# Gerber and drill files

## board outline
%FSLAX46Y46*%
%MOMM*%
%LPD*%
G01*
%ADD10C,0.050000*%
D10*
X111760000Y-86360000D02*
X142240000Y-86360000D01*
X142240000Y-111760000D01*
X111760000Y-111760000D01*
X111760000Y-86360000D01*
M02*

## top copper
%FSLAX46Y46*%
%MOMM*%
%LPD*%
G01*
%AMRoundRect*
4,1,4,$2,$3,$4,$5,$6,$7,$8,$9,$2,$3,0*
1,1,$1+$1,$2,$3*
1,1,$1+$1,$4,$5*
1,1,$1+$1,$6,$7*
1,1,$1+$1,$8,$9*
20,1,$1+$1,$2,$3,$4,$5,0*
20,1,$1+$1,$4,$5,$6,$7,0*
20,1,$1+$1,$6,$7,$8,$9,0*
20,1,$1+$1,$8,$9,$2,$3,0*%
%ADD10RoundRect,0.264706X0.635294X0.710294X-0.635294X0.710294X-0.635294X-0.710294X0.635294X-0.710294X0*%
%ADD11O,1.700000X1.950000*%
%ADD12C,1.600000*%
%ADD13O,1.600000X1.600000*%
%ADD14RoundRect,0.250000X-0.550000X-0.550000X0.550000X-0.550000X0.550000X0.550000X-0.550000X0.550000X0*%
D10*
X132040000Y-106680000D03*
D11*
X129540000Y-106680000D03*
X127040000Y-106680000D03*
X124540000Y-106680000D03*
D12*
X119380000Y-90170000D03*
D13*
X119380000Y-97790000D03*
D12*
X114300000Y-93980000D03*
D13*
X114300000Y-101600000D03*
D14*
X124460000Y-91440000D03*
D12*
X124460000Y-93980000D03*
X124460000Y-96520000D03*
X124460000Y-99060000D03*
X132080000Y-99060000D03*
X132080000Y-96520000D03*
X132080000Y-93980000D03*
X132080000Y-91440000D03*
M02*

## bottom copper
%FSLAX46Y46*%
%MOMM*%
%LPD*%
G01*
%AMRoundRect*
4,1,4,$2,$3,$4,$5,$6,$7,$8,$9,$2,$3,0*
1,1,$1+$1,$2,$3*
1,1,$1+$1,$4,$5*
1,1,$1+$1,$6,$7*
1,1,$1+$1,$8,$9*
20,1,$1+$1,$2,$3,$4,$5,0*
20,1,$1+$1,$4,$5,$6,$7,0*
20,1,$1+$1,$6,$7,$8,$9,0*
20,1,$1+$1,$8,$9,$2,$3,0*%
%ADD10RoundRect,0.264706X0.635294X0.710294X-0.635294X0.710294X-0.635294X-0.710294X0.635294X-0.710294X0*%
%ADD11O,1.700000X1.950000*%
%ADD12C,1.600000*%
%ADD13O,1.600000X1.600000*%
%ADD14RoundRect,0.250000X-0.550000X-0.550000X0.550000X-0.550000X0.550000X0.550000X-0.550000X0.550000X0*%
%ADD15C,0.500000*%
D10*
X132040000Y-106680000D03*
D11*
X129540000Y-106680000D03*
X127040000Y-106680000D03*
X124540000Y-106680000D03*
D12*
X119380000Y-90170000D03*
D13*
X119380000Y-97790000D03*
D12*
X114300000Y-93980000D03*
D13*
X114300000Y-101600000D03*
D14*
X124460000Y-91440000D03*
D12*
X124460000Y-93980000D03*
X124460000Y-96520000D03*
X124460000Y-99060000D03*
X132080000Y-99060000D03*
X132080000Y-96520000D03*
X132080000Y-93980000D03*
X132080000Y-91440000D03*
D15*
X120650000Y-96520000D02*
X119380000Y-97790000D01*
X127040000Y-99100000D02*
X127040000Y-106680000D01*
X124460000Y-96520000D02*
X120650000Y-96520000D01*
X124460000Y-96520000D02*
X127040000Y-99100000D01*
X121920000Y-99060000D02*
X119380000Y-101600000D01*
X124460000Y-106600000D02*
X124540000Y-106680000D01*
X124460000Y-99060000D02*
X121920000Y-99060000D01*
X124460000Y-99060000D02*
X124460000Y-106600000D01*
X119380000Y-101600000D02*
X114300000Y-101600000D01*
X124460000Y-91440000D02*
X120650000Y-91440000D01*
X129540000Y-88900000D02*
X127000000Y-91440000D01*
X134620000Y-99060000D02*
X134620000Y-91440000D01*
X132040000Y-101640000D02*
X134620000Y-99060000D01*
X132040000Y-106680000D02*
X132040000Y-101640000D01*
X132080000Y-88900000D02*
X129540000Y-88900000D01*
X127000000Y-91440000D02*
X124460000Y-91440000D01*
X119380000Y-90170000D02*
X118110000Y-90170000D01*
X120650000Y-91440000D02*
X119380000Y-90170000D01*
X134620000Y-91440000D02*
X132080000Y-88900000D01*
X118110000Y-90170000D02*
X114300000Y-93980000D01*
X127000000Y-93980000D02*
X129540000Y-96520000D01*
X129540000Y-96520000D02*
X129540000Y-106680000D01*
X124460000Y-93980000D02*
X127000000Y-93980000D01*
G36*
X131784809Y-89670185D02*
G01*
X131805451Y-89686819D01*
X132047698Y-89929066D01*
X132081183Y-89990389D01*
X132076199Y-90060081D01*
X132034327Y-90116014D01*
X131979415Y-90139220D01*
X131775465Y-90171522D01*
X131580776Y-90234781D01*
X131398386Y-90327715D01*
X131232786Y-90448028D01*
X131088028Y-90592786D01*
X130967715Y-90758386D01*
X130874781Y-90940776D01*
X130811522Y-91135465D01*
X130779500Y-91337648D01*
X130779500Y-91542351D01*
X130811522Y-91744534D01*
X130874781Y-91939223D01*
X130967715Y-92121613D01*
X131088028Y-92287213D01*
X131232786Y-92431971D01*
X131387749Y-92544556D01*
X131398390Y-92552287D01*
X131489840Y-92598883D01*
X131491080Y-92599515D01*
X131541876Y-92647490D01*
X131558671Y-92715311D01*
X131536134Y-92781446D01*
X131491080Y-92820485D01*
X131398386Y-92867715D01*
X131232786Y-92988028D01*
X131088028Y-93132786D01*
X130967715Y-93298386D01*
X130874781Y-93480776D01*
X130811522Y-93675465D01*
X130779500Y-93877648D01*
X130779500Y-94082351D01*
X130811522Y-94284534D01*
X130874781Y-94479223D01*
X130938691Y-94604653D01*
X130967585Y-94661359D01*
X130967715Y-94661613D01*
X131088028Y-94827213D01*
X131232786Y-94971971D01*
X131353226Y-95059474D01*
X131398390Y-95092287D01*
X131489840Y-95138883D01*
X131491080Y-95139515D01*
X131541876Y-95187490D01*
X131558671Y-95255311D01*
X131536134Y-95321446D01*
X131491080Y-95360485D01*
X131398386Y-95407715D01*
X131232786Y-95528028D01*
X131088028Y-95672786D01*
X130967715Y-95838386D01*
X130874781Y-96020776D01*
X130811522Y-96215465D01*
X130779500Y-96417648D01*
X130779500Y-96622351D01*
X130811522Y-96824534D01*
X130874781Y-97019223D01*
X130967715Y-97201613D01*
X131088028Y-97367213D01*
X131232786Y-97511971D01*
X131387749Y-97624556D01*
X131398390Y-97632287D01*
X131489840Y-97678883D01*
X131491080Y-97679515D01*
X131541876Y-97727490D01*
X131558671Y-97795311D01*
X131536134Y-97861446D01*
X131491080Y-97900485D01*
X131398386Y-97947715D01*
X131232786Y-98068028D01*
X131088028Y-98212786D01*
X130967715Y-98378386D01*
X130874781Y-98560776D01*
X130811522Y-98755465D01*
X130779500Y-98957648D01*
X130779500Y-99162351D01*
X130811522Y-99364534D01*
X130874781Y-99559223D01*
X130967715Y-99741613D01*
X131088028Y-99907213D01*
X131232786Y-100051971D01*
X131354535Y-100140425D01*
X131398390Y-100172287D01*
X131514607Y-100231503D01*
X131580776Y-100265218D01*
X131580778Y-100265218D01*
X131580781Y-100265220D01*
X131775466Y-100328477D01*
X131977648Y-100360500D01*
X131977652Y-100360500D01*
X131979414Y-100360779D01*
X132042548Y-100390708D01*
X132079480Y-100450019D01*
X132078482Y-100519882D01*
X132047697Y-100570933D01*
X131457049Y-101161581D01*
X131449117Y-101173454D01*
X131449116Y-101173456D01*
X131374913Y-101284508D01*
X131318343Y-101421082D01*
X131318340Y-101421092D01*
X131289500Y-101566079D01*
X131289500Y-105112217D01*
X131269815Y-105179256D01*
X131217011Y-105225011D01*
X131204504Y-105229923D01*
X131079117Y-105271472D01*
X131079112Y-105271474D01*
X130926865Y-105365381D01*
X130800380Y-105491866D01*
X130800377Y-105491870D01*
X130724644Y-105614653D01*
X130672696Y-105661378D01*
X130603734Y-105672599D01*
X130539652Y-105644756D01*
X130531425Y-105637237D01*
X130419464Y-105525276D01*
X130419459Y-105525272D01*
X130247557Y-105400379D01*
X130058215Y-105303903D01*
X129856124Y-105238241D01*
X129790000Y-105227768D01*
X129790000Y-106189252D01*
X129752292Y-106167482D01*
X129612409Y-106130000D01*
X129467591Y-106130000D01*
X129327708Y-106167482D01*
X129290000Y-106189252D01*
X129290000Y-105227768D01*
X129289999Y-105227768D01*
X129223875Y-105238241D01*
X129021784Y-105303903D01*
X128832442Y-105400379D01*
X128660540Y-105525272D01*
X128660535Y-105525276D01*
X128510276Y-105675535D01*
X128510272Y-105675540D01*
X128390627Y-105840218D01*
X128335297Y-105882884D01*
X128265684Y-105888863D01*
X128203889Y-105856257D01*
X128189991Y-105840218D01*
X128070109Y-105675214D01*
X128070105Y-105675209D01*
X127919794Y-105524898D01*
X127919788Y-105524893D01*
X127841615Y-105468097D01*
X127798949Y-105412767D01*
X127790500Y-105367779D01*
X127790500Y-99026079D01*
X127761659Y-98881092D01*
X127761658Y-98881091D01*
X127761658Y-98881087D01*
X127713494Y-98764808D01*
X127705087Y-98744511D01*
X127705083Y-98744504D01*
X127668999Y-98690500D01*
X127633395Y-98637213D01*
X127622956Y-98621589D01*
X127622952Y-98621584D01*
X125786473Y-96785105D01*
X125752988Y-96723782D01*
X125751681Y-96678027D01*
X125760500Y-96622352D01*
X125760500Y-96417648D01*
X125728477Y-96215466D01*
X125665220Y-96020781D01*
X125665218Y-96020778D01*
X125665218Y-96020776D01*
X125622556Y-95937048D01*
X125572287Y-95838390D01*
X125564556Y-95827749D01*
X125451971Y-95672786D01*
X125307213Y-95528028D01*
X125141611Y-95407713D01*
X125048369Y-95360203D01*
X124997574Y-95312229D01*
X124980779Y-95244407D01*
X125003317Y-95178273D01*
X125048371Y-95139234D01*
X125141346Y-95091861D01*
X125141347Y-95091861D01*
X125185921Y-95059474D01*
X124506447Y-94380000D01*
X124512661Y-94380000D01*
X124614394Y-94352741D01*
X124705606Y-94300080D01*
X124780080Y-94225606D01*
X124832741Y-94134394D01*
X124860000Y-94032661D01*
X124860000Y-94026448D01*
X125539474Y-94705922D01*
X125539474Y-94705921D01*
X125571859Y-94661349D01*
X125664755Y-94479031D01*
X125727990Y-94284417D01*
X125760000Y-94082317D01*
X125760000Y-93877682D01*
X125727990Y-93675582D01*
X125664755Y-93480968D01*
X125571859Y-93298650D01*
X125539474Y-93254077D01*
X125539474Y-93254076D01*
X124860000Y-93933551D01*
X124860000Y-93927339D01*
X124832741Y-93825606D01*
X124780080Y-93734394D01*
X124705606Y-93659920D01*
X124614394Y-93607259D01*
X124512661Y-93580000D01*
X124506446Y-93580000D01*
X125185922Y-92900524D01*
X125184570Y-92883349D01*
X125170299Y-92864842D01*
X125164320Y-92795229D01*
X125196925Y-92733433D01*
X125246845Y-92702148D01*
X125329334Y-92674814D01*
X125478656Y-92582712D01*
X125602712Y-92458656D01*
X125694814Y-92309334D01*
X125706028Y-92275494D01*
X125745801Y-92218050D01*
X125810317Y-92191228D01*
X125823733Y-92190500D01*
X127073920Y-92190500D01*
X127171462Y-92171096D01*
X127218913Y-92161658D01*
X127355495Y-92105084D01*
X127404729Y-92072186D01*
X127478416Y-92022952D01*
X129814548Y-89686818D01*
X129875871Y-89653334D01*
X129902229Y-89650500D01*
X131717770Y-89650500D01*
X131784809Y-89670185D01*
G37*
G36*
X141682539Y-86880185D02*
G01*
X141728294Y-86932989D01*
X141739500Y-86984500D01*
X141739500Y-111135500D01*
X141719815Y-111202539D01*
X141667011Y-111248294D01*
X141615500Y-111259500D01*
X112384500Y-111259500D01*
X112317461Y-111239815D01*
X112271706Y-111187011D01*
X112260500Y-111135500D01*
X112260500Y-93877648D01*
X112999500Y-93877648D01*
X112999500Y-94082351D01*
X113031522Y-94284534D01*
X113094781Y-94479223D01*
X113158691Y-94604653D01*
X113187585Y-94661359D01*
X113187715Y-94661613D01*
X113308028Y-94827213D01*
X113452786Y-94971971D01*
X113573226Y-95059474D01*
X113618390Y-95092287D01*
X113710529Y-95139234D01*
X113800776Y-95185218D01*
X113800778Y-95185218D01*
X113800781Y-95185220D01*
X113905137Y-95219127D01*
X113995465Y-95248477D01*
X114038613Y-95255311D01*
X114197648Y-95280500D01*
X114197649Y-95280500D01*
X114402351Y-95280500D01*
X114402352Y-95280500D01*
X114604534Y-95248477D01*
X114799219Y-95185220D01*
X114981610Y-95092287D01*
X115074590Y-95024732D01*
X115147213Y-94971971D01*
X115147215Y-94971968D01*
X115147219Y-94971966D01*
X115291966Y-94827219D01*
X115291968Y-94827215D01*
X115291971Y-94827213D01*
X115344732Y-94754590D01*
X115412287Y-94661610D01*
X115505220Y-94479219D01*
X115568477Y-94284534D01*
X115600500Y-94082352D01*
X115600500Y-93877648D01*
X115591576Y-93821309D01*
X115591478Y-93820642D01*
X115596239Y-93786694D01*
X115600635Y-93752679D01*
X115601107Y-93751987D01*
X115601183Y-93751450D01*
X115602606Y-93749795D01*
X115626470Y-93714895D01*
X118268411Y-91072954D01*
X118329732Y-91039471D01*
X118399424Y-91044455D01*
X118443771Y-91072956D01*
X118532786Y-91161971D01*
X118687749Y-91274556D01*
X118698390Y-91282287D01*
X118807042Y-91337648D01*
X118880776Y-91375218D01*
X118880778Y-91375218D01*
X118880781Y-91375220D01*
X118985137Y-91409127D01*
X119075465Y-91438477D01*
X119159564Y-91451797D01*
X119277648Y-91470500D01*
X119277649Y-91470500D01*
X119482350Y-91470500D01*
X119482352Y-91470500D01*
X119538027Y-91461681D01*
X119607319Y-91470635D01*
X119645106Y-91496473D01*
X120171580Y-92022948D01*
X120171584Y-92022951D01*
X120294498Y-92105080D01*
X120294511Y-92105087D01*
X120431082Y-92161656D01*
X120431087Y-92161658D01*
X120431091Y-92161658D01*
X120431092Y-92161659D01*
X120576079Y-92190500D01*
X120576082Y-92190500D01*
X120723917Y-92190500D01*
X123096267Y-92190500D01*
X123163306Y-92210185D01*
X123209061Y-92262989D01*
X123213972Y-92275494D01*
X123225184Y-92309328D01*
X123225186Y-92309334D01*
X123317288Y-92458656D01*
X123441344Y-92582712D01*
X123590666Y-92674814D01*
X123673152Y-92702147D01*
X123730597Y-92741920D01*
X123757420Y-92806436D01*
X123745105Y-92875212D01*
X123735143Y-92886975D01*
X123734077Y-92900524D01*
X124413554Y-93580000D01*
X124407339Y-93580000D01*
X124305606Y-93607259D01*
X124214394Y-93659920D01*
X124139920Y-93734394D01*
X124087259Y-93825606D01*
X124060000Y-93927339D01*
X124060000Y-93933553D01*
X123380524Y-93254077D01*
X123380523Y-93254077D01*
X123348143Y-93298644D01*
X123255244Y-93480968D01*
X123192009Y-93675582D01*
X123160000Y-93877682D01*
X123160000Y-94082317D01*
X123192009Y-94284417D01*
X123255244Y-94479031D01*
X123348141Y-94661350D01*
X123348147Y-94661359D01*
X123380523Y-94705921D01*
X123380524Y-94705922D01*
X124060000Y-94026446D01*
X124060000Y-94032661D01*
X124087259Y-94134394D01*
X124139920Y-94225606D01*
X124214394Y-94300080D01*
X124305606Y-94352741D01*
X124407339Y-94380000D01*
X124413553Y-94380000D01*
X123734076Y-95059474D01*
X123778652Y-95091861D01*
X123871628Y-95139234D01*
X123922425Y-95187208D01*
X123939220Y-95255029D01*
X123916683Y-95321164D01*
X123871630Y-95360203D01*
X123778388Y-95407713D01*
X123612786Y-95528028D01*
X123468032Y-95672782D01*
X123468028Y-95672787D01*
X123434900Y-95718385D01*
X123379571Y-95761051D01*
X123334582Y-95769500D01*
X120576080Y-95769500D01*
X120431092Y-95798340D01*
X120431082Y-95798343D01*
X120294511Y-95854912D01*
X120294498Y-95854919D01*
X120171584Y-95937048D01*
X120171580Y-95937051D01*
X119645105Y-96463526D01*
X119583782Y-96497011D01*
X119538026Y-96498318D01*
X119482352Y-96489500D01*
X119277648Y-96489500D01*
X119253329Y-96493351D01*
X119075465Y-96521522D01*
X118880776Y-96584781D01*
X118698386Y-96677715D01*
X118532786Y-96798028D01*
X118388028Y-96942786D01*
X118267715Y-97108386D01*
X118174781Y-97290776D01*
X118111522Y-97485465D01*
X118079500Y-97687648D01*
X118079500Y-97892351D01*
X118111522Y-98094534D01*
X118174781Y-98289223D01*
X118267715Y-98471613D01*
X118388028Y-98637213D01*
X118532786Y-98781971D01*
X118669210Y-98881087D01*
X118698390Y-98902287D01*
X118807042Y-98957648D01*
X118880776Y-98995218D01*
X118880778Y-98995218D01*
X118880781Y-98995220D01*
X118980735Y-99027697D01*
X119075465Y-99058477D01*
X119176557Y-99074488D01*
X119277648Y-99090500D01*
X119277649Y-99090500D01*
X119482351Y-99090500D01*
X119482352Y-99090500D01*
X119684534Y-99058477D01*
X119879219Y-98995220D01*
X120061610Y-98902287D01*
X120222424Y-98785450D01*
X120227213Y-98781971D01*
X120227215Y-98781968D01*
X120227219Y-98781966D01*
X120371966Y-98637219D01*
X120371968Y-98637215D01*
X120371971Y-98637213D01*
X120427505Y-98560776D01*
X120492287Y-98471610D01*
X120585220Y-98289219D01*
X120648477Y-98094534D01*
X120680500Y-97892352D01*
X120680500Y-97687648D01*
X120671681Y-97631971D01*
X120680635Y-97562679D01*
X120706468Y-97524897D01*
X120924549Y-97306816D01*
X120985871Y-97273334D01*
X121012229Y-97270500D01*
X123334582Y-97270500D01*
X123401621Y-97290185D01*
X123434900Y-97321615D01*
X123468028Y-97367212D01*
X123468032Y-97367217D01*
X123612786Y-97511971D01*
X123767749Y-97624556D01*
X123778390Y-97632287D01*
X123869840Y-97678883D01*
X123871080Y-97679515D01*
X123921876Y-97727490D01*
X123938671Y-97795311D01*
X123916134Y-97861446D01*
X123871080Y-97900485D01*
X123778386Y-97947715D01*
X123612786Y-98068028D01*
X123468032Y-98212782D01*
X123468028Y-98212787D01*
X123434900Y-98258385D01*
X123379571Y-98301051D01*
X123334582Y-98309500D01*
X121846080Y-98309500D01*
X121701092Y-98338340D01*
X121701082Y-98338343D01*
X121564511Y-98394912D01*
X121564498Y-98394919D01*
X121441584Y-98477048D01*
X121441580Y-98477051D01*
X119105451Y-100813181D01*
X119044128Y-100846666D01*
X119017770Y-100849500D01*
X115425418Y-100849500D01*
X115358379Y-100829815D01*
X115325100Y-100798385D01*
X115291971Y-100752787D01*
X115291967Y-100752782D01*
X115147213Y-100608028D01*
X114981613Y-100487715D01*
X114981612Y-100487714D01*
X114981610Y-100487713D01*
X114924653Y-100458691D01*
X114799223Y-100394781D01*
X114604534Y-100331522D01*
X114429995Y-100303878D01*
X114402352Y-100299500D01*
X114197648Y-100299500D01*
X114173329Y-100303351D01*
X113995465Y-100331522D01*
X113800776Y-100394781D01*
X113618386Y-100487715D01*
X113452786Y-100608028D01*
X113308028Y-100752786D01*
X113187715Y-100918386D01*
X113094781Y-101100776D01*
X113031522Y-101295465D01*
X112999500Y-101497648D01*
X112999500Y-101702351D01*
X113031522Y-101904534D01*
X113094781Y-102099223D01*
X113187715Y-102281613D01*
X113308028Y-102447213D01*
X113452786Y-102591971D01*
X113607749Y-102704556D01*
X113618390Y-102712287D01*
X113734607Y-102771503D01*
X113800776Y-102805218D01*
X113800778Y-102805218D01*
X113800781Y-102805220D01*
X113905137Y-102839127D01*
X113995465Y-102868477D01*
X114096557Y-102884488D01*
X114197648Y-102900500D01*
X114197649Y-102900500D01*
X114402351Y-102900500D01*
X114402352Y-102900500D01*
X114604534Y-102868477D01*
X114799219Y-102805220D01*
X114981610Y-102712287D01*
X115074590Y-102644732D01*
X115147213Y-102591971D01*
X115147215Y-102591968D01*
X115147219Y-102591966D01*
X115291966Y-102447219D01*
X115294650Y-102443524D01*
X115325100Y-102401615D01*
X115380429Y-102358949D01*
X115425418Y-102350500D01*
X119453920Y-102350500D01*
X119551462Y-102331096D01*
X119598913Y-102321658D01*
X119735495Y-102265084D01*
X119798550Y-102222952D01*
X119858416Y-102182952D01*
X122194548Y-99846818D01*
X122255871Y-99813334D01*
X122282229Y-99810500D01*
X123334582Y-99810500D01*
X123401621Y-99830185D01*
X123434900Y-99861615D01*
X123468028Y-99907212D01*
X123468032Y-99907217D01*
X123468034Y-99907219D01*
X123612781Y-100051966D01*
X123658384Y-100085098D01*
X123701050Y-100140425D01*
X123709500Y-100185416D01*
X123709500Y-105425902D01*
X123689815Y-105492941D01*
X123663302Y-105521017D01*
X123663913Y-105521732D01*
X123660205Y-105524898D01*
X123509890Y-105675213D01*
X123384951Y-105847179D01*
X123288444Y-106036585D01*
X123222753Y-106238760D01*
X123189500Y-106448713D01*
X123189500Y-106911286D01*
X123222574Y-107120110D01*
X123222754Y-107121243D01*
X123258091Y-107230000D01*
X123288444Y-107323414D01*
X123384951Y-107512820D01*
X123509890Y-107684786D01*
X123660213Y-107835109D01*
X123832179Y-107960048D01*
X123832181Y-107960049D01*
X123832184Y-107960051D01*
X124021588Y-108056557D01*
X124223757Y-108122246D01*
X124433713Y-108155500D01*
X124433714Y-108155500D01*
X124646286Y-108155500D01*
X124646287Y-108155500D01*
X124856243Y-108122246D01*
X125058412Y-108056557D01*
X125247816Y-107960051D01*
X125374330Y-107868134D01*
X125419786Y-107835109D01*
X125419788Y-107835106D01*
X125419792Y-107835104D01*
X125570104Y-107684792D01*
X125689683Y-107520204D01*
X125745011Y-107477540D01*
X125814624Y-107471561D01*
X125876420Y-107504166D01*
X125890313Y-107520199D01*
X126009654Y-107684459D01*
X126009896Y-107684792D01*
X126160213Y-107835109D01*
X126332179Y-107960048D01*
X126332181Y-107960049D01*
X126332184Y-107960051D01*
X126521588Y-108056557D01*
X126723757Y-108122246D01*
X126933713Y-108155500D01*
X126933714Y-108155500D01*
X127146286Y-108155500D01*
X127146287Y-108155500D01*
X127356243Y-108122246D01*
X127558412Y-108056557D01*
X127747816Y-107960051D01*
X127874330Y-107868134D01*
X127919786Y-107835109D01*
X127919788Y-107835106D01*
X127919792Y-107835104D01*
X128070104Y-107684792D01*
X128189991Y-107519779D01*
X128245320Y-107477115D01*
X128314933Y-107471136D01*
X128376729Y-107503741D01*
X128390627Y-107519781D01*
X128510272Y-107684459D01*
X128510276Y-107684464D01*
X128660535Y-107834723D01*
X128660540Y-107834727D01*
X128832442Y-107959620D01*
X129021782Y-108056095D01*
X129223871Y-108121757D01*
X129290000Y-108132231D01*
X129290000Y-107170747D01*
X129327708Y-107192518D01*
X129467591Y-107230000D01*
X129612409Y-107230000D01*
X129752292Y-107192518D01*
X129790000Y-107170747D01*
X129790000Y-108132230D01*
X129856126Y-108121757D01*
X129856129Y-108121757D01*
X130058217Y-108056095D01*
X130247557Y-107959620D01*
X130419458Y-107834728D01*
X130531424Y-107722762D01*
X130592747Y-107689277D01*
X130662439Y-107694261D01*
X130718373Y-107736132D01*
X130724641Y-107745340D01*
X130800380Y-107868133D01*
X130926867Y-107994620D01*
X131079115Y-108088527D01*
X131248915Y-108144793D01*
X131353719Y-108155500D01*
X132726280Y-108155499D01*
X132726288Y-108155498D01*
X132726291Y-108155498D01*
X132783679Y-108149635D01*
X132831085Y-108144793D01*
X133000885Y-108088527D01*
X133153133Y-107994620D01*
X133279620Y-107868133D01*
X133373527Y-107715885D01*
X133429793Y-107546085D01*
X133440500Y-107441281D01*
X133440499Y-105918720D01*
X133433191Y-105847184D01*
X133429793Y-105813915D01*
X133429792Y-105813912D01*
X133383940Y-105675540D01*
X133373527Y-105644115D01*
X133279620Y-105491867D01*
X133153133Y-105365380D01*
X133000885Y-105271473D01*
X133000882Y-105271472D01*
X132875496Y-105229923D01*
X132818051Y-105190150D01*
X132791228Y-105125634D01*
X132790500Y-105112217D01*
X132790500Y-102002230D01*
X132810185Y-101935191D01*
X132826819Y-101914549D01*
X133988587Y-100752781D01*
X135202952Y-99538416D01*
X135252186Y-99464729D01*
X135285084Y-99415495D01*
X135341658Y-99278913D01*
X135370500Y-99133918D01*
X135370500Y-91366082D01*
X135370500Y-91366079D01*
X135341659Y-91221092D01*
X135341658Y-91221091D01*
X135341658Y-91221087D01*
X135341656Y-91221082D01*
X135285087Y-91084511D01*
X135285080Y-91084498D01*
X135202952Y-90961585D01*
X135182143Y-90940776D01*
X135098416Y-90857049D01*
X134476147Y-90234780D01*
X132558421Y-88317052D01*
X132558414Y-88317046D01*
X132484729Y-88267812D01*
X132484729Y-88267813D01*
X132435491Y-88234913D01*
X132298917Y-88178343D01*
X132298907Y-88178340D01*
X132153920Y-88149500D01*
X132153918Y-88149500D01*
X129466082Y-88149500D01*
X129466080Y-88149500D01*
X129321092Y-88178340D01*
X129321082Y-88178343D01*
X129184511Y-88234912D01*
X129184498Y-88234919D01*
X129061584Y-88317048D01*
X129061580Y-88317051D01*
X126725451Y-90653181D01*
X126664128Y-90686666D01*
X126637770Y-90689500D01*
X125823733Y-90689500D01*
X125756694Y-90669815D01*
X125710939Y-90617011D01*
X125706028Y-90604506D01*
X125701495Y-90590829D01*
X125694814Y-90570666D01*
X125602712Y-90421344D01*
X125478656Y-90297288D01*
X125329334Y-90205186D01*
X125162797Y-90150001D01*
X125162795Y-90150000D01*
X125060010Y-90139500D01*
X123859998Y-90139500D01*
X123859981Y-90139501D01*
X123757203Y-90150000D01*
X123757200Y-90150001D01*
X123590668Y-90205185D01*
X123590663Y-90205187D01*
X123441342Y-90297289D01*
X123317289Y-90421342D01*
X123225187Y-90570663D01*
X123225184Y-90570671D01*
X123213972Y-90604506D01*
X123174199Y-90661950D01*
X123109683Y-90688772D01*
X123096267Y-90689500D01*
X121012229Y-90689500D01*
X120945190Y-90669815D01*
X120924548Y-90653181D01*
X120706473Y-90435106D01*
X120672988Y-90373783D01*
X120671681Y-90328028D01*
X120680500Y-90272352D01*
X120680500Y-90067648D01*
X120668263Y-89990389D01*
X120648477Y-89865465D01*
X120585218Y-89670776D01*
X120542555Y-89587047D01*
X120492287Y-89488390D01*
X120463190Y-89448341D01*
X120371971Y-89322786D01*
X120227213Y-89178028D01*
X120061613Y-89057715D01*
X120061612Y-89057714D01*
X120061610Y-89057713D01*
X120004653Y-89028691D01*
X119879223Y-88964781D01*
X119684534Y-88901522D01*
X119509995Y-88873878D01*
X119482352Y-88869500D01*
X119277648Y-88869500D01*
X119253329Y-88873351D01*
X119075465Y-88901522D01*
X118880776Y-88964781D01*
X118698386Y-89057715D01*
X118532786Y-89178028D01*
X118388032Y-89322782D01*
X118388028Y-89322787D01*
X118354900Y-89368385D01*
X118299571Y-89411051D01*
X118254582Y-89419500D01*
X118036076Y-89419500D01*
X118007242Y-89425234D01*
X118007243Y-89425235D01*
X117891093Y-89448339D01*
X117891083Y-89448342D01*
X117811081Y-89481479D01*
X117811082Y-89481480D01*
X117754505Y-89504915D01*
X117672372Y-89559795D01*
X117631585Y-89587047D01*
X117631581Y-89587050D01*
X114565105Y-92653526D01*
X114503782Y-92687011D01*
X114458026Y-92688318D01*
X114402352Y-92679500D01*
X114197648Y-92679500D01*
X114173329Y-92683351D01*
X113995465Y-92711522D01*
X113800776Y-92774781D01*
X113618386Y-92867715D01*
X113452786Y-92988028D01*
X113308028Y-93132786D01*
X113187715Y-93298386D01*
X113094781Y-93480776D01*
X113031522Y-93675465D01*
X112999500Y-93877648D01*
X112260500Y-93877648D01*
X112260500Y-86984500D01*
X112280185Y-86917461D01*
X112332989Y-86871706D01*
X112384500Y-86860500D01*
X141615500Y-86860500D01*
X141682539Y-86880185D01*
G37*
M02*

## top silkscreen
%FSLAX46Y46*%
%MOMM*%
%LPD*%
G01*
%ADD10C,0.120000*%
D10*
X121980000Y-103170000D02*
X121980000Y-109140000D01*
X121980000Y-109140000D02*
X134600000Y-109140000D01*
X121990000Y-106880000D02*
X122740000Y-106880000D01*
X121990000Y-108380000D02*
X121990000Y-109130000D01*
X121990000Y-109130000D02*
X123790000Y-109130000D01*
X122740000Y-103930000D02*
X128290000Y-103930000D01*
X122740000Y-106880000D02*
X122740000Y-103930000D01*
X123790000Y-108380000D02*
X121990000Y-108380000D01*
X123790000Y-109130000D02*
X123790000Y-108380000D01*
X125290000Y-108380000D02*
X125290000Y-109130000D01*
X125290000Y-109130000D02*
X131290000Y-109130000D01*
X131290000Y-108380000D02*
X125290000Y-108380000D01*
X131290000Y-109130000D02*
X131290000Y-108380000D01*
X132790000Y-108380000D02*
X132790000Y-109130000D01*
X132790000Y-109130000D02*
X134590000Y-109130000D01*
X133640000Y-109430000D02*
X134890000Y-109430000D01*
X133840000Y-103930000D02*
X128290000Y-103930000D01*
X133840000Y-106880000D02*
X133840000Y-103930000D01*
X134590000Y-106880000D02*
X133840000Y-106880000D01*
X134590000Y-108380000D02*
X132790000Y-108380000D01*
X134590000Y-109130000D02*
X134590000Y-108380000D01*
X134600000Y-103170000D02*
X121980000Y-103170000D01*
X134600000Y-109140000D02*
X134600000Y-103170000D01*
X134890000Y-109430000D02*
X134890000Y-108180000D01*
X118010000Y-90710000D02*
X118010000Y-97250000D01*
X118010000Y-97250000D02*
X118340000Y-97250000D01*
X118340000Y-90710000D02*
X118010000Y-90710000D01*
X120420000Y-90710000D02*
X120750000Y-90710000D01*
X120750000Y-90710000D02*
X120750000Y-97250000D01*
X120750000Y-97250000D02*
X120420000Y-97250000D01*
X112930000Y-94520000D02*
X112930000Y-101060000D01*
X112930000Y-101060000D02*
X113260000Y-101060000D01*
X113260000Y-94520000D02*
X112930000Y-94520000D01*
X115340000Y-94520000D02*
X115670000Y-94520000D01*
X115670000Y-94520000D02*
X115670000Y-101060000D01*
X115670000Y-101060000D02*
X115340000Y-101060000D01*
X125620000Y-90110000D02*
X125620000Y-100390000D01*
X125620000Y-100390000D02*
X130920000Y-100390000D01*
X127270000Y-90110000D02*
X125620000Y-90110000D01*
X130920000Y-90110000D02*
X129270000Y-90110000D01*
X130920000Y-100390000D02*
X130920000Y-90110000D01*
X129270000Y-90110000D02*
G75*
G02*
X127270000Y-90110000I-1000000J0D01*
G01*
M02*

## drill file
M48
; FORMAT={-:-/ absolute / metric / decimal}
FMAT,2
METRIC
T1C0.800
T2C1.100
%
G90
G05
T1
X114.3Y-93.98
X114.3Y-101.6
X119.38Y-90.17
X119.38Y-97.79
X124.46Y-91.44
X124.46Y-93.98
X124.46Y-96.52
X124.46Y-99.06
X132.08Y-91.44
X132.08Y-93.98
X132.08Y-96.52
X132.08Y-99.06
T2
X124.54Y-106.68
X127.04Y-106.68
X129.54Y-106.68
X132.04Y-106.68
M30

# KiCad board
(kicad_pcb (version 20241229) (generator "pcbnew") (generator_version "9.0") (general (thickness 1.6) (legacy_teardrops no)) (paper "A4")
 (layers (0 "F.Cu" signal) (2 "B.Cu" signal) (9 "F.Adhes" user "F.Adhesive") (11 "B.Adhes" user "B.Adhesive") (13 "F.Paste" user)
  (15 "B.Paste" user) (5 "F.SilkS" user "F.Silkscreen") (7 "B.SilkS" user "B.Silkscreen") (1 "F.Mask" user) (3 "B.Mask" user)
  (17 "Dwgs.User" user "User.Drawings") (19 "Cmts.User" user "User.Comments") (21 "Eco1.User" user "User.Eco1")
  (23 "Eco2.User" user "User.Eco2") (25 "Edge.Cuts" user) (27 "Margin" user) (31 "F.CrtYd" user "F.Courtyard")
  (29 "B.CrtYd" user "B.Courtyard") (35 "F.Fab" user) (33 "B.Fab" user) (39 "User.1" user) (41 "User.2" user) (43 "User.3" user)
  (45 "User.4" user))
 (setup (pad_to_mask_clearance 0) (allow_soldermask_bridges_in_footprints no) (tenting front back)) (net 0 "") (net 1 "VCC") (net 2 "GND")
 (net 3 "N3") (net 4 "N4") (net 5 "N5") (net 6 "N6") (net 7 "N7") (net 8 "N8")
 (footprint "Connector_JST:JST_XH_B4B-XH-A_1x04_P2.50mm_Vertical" (layer "F.Cu") (at 132.04 106.68 180)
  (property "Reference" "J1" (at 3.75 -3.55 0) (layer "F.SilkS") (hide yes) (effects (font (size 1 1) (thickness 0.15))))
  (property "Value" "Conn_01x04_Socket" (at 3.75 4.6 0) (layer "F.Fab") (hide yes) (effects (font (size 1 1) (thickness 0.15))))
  (fp_line (start 10.06 3.51) (end 10.06 -2.46) (stroke (width 0.12) (type solid)) (layer "F.SilkS"))
  (fp_line (start 10.06 -2.46) (end -2.56 -2.46) (stroke (width 0.12) (type solid)) (layer "F.SilkS"))
  (fp_line (start 10.05 -0.2) (end 9.3 -0.2) (stroke (width 0.12) (type solid)) (layer "F.SilkS"))
  (fp_line (start 10.05 -1.7) (end 10.05 -2.45) (stroke (width 0.12) (type solid)) (layer "F.SilkS"))
  (fp_line (start 10.05 -2.45) (end 8.25 -2.45) (stroke (width 0.12) (type solid)) (layer "F.SilkS"))
  (fp_line (start 9.3 2.75) (end 3.75 2.75) (stroke (width 0.12) (type solid)) (layer "F.SilkS"))
  (fp_line (start 9.3 -0.2) (end 9.3 2.75) (stroke (width 0.12) (type solid)) (layer "F.SilkS"))
  (fp_line (start 8.25 -1.7) (end 10.05 -1.7) (stroke (width 0.12) (type solid)) (layer "F.SilkS"))
  (fp_line (start 8.25 -2.45) (end 8.25 -1.7) (stroke (width 0.12) (type solid)) (layer "F.SilkS"))
  (fp_line (start 6.75 -1.7) (end 6.75 -2.45) (stroke (width 0.12) (type solid)) (layer "F.SilkS"))
  (fp_line (start 6.75 -2.45) (end 0.75 -2.45) (stroke (width 0.12) (type solid)) (layer "F.SilkS"))
  (fp_line (start 0.75 -1.7) (end 6.75 -1.7) (stroke (width 0.12) (type solid)) (layer "F.SilkS"))
  (fp_line (start 0.75 -2.45) (end 0.75 -1.7) (stroke (width 0.12) (type solid)) (layer "F.SilkS"))
  (fp_line (start -0.75 -1.7) (end -0.75 -2.45) (stroke (width 0.12) (type solid)) (layer "F.SilkS"))
  (fp_line (start -0.75 -2.45) (end -2.55 -2.45) (stroke (width 0.12) (type solid)) (layer "F.SilkS"))
  (fp_line (start -1.6 -2.75) (end -2.85 -2.75) (stroke (width 0.12) (type solid)) (layer "F.SilkS"))
  (fp_line (start -1.8 2.75) (end 3.75 2.75) (stroke (width 0.12) (type solid)) (layer "F.SilkS"))
  (fp_line (start -1.8 -0.2) (end -1.8 2.75) (stroke (width 0.12) (type solid)) (layer "F.SilkS"))
  (fp_line (start -2.55 -0.2) (end -1.8 -0.2) (stroke (width 0.12) (type solid)) (layer "F.SilkS"))
  (fp_line (start -2.55 -1.7) (end -0.75 -1.7) (stroke (width 0.12) (type solid)) (layer "F.SilkS"))
  (fp_line (start -2.55 -2.45) (end -2.55 -1.7) (stroke (width 0.12) (type solid)) (layer "F.SilkS"))
  (fp_line (start -2.56 3.51) (end 10.06 3.51) (stroke (width 0.12) (type solid)) (layer "F.SilkS"))
  (fp_line (start -2.56 -2.46) (end -2.56 3.51) (stroke (width 0.12) (type solid)) (layer "F.SilkS"))
  (fp_line (start -2.85 -2.75) (end -2.85 -1.5) (stroke (width 0.12) (type solid)) (layer "F.SilkS"))
  (pad "1" thru_hole roundrect (at 0 0 180) (size 1.8 1.95) (drill 1.1) (layers "*.Cu" "*.Mask") (remove_unused_layers no)
   (roundrect_rratio 0.147059) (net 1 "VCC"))
  (pad "2" thru_hole oval (at 2.5 0 180) (size 1.7 1.95) (drill 1.1) (layers "*.Cu" "*.Mask") (remove_unused_layers no) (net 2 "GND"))
  (pad "3" thru_hole oval (at 5 0 180) (size 1.7 1.95) (drill 1.1) (layers "*.Cu" "*.Mask") (remove_unused_layers no) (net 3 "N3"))
  (pad "4" thru_hole oval (at 7.5 0 180) (size 1.7 1.95) (drill 1.1) (layers "*.Cu" "*.Mask") (remove_unused_layers no) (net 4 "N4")))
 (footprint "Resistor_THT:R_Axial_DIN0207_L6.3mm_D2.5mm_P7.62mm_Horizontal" (layer "F.Cu") (at 119.38 90.17 -90)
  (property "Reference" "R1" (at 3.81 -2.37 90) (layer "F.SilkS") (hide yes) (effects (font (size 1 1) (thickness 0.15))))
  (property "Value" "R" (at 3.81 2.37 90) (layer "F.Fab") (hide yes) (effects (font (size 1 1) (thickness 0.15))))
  (fp_line (start 0.54 1.37) (end 7.08 1.37) (stroke (width 0.12) (type solid)) (layer "F.SilkS"))
  (fp_line (start 7.08 1.37) (end 7.08 1.04) (stroke (width 0.12) (type solid)) (layer "F.SilkS"))
  (fp_line (start 0.54 1.04) (end 0.54 1.37) (stroke (width 0.12) (type solid)) (layer "F.SilkS"))
  (fp_line (start 0.54 -1.04) (end 0.54 -1.37) (stroke (width 0.12) (type solid)) (layer "F.SilkS"))
  (fp_line (start 0.54 -1.37) (end 7.08 -1.37) (stroke (width 0.12) (type solid)) (layer "F.SilkS"))
  (fp_line (start 7.08 -1.37) (end 7.08 -1.04) (stroke (width 0.12) (type solid)) (layer "F.SilkS"))
  (pad "1" thru_hole circle (at 0 0 270) (size 1.6 1.6) (drill 0.8) (layers "*.Cu" "*.Mask") (remove_unused_layers no) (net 1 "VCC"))
  (pad "2" thru_hole oval (at 7.62 0 270) (size 1.6 1.6) (drill 0.8) (layers "*.Cu" "*.Mask") (remove_unused_layers no) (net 3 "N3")))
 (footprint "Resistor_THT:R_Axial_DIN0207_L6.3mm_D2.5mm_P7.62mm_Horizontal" (layer "F.Cu") (at 114.3 93.98 -90)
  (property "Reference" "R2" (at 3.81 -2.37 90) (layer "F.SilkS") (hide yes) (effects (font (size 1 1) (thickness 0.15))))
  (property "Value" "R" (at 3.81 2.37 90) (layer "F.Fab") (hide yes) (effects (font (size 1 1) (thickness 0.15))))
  (fp_line (start 0.54 1.37) (end 7.08 1.37) (stroke (width 0.12) (type solid)) (layer "F.SilkS"))
  (fp_line (start 7.08 1.37) (end 7.08 1.04) (stroke (width 0.12) (type solid)) (layer "F.SilkS"))
  (fp_line (start 0.54 1.04) (end 0.54 1.37) (stroke (width 0.12) (type solid)) (layer "F.SilkS"))
  (fp_line (start 0.54 -1.04) (end 0.54 -1.37) (stroke (width 0.12) (type solid)) (layer "F.SilkS"))
  (fp_line (start 0.54 -1.37) (end 7.08 -1.37) (stroke (width 0.12) (type solid)) (layer "F.SilkS"))
  (fp_line (start 7.08 -1.37) (end 7.08 -1.04) (stroke (width 0.12) (type solid)) (layer "F.SilkS"))
  (pad "1" thru_hole circle (at 0 0 270) (size 1.6 1.6) (drill 0.8) (layers "*.Cu" "*.Mask") (remove_unused_layers no) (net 1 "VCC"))
  (pad "2" thru_hole oval (at 7.62 0 270) (size 1.6 1.6) (drill 0.8) (layers "*.Cu" "*.Mask") (remove_unused_layers no) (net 4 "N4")))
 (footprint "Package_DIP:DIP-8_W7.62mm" (layer "F.Cu") (at 124.46 91.44)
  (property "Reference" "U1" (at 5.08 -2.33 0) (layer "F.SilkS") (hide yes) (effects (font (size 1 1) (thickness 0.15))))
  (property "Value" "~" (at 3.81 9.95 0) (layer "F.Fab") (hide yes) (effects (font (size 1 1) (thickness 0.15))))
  (fp_line (start 1.16 -1.33) (end 1.16 8.95) (stroke (width 0.12) (type solid)) (layer "F.SilkS"))
  (fp_line (start 1.16 8.95) (end 6.46 8.95) (stroke (width 0.12) (type solid)) (layer "F.SilkS"))
  (fp_line (start 2.81 -1.33) (end 1.16 -1.33) (stroke (width 0.12) (type solid)) (layer "F.SilkS"))
  (fp_line (start 6.46 -1.33) (end 4.81 -1.33) (stroke (width 0.12) (type solid)) (layer "F.SilkS"))
  (fp_line (start 6.46 8.95) (end 6.46 -1.33) (stroke (width 0.12) (type solid)) (layer "F.SilkS"))
  (fp_arc (start 4.81 -1.33) (mid 3.81 -0.33) (end 2.81 -1.33) (stroke (width 0.12) (type solid)) (layer "F.SilkS"))
  (pad "1" thru_hole roundrect (at 0 0) (size 1.6 1.6) (drill 0.8) (layers "*.Cu" "*.Mask") (remove_unused_layers no)
   (roundrect_rratio 0.15625) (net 1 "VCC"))
  (pad "2" thru_hole circle (at 0 2.54) (size 1.6 1.6) (drill 0.8) (layers "*.Cu" "*.Mask") (remove_unused_layers no) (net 2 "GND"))
  (pad "3" thru_hole circle (at 0 5.08) (size 1.6 1.6) (drill 0.8) (layers "*.Cu" "*.Mask") (remove_unused_layers no) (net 3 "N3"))
  (pad "4" thru_hole circle (at 0 7.62) (size 1.6 1.6) (drill 0.8) (layers "*.Cu" "*.Mask") (remove_unused_layers no) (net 4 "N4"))
  (pad "5" thru_hole circle (at 7.62 7.62) (size 1.6 1.6) (drill 0.8) (layers "*.Cu" "*.Mask") (remove_unused_layers no) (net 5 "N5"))
  (pad "6" thru_hole circle (at 7.62 5.08) (size 1.6 1.6) (drill 0.8) (layers "*.Cu" "*.Mask") (remove_unused_layers no) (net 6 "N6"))
  (pad "7" thru_hole circle (at 7.62 2.54) (size 1.6 1.6) (drill 0.8) (layers "*.Cu" "*.Mask") (remove_unused_layers no) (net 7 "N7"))
  (pad "8" thru_hole circle (at 7.62 0) (size 1.6 1.6) (drill 0.8) (layers "*.Cu" "*.Mask") (remove_unused_layers no) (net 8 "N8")))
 (gr_rect (start 111.76 86.36) (end 142.24 111.76) (stroke (width 0.05) (type solid)) (fill no) (layer "Edge.Cuts"))
 (segment (start 120.65 96.52) (end 119.38 97.79) (width 0.5) (layer "B.Cu") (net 3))
 (segment (start 127.04 99.1) (end 127.04 106.68) (width 0.5) (layer "B.Cu") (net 3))
 (segment (start 124.46 96.52) (end 120.65 96.52) (width 0.5) (layer "B.Cu") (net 3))
 (segment (start 124.46 96.52) (end 127.04 99.1) (width 0.5) (layer "B.Cu") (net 3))
 (segment (start 121.92 99.06) (end 119.38 101.6) (width 0.5) (layer "B.Cu") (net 4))
 (segment (start 124.46 106.6) (end 124.54 106.68) (width 0.5) (layer "B.Cu") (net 4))
 (segment (start 124.46 99.06) (end 121.92 99.06) (width 0.5) (layer "B.Cu") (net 4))
 (segment (start 124.46 99.06) (end 124.46 106.6) (width 0.5) (layer "B.Cu") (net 4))
 (segment (start 119.38 101.6) (end 114.3 101.6) (width 0.5) (layer "B.Cu") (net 4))
 (segment (start 124.46 91.44) (end 120.65 91.44) (width 0.5) (layer "B.Cu") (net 1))
 (segment (start 129.54 88.9) (end 127 91.44) (width 0.5) (layer "B.Cu") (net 1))
 (segment (start 134.62 99.06) (end 134.62 91.44) (width 0.5) (layer "B.Cu") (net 1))
 (segment (start 132.04 101.64) (end 134.62 99.06) (width 0.5) (layer "B.Cu") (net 1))
 (segment (start 132.04 106.68) (end 132.04 101.64) (width 0.5) (layer "B.Cu") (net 1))
 (segment (start 132.08 88.9) (end 129.54 88.9) (width 0.5) (layer "B.Cu") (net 1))
 (segment (start 127 91.44) (end 124.46 91.44) (width 0.5) (layer "B.Cu") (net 1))
 (segment (start 119.38 90.17) (end 118.11 90.17) (width 0.5) (layer "B.Cu") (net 1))
 (segment (start 120.65 91.44) (end 119.38 90.17) (width 0.5) (layer "B.Cu") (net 1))
 (segment (start 134.62 91.44) (end 132.08 88.9) (width 0.5) (layer "B.Cu") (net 1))
 (segment (start 118.11 90.17) (end 114.3 93.98) (width 0.5) (layer "B.Cu") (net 1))
 (segment (start 127 93.98) (end 129.54 96.52) (width 0.5) (layer "B.Cu") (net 2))
 (segment (start 129.54 96.52) (end 129.54 106.68) (width 0.5) (layer "B.Cu") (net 2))
 (segment (start 124.46 93.98) (end 127 93.98) (width 0.5) (layer "B.Cu") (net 2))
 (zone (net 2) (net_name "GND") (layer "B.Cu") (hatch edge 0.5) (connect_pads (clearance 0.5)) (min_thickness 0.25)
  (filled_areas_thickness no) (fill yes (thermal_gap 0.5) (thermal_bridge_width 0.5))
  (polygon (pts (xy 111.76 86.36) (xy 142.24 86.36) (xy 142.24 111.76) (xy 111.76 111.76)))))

